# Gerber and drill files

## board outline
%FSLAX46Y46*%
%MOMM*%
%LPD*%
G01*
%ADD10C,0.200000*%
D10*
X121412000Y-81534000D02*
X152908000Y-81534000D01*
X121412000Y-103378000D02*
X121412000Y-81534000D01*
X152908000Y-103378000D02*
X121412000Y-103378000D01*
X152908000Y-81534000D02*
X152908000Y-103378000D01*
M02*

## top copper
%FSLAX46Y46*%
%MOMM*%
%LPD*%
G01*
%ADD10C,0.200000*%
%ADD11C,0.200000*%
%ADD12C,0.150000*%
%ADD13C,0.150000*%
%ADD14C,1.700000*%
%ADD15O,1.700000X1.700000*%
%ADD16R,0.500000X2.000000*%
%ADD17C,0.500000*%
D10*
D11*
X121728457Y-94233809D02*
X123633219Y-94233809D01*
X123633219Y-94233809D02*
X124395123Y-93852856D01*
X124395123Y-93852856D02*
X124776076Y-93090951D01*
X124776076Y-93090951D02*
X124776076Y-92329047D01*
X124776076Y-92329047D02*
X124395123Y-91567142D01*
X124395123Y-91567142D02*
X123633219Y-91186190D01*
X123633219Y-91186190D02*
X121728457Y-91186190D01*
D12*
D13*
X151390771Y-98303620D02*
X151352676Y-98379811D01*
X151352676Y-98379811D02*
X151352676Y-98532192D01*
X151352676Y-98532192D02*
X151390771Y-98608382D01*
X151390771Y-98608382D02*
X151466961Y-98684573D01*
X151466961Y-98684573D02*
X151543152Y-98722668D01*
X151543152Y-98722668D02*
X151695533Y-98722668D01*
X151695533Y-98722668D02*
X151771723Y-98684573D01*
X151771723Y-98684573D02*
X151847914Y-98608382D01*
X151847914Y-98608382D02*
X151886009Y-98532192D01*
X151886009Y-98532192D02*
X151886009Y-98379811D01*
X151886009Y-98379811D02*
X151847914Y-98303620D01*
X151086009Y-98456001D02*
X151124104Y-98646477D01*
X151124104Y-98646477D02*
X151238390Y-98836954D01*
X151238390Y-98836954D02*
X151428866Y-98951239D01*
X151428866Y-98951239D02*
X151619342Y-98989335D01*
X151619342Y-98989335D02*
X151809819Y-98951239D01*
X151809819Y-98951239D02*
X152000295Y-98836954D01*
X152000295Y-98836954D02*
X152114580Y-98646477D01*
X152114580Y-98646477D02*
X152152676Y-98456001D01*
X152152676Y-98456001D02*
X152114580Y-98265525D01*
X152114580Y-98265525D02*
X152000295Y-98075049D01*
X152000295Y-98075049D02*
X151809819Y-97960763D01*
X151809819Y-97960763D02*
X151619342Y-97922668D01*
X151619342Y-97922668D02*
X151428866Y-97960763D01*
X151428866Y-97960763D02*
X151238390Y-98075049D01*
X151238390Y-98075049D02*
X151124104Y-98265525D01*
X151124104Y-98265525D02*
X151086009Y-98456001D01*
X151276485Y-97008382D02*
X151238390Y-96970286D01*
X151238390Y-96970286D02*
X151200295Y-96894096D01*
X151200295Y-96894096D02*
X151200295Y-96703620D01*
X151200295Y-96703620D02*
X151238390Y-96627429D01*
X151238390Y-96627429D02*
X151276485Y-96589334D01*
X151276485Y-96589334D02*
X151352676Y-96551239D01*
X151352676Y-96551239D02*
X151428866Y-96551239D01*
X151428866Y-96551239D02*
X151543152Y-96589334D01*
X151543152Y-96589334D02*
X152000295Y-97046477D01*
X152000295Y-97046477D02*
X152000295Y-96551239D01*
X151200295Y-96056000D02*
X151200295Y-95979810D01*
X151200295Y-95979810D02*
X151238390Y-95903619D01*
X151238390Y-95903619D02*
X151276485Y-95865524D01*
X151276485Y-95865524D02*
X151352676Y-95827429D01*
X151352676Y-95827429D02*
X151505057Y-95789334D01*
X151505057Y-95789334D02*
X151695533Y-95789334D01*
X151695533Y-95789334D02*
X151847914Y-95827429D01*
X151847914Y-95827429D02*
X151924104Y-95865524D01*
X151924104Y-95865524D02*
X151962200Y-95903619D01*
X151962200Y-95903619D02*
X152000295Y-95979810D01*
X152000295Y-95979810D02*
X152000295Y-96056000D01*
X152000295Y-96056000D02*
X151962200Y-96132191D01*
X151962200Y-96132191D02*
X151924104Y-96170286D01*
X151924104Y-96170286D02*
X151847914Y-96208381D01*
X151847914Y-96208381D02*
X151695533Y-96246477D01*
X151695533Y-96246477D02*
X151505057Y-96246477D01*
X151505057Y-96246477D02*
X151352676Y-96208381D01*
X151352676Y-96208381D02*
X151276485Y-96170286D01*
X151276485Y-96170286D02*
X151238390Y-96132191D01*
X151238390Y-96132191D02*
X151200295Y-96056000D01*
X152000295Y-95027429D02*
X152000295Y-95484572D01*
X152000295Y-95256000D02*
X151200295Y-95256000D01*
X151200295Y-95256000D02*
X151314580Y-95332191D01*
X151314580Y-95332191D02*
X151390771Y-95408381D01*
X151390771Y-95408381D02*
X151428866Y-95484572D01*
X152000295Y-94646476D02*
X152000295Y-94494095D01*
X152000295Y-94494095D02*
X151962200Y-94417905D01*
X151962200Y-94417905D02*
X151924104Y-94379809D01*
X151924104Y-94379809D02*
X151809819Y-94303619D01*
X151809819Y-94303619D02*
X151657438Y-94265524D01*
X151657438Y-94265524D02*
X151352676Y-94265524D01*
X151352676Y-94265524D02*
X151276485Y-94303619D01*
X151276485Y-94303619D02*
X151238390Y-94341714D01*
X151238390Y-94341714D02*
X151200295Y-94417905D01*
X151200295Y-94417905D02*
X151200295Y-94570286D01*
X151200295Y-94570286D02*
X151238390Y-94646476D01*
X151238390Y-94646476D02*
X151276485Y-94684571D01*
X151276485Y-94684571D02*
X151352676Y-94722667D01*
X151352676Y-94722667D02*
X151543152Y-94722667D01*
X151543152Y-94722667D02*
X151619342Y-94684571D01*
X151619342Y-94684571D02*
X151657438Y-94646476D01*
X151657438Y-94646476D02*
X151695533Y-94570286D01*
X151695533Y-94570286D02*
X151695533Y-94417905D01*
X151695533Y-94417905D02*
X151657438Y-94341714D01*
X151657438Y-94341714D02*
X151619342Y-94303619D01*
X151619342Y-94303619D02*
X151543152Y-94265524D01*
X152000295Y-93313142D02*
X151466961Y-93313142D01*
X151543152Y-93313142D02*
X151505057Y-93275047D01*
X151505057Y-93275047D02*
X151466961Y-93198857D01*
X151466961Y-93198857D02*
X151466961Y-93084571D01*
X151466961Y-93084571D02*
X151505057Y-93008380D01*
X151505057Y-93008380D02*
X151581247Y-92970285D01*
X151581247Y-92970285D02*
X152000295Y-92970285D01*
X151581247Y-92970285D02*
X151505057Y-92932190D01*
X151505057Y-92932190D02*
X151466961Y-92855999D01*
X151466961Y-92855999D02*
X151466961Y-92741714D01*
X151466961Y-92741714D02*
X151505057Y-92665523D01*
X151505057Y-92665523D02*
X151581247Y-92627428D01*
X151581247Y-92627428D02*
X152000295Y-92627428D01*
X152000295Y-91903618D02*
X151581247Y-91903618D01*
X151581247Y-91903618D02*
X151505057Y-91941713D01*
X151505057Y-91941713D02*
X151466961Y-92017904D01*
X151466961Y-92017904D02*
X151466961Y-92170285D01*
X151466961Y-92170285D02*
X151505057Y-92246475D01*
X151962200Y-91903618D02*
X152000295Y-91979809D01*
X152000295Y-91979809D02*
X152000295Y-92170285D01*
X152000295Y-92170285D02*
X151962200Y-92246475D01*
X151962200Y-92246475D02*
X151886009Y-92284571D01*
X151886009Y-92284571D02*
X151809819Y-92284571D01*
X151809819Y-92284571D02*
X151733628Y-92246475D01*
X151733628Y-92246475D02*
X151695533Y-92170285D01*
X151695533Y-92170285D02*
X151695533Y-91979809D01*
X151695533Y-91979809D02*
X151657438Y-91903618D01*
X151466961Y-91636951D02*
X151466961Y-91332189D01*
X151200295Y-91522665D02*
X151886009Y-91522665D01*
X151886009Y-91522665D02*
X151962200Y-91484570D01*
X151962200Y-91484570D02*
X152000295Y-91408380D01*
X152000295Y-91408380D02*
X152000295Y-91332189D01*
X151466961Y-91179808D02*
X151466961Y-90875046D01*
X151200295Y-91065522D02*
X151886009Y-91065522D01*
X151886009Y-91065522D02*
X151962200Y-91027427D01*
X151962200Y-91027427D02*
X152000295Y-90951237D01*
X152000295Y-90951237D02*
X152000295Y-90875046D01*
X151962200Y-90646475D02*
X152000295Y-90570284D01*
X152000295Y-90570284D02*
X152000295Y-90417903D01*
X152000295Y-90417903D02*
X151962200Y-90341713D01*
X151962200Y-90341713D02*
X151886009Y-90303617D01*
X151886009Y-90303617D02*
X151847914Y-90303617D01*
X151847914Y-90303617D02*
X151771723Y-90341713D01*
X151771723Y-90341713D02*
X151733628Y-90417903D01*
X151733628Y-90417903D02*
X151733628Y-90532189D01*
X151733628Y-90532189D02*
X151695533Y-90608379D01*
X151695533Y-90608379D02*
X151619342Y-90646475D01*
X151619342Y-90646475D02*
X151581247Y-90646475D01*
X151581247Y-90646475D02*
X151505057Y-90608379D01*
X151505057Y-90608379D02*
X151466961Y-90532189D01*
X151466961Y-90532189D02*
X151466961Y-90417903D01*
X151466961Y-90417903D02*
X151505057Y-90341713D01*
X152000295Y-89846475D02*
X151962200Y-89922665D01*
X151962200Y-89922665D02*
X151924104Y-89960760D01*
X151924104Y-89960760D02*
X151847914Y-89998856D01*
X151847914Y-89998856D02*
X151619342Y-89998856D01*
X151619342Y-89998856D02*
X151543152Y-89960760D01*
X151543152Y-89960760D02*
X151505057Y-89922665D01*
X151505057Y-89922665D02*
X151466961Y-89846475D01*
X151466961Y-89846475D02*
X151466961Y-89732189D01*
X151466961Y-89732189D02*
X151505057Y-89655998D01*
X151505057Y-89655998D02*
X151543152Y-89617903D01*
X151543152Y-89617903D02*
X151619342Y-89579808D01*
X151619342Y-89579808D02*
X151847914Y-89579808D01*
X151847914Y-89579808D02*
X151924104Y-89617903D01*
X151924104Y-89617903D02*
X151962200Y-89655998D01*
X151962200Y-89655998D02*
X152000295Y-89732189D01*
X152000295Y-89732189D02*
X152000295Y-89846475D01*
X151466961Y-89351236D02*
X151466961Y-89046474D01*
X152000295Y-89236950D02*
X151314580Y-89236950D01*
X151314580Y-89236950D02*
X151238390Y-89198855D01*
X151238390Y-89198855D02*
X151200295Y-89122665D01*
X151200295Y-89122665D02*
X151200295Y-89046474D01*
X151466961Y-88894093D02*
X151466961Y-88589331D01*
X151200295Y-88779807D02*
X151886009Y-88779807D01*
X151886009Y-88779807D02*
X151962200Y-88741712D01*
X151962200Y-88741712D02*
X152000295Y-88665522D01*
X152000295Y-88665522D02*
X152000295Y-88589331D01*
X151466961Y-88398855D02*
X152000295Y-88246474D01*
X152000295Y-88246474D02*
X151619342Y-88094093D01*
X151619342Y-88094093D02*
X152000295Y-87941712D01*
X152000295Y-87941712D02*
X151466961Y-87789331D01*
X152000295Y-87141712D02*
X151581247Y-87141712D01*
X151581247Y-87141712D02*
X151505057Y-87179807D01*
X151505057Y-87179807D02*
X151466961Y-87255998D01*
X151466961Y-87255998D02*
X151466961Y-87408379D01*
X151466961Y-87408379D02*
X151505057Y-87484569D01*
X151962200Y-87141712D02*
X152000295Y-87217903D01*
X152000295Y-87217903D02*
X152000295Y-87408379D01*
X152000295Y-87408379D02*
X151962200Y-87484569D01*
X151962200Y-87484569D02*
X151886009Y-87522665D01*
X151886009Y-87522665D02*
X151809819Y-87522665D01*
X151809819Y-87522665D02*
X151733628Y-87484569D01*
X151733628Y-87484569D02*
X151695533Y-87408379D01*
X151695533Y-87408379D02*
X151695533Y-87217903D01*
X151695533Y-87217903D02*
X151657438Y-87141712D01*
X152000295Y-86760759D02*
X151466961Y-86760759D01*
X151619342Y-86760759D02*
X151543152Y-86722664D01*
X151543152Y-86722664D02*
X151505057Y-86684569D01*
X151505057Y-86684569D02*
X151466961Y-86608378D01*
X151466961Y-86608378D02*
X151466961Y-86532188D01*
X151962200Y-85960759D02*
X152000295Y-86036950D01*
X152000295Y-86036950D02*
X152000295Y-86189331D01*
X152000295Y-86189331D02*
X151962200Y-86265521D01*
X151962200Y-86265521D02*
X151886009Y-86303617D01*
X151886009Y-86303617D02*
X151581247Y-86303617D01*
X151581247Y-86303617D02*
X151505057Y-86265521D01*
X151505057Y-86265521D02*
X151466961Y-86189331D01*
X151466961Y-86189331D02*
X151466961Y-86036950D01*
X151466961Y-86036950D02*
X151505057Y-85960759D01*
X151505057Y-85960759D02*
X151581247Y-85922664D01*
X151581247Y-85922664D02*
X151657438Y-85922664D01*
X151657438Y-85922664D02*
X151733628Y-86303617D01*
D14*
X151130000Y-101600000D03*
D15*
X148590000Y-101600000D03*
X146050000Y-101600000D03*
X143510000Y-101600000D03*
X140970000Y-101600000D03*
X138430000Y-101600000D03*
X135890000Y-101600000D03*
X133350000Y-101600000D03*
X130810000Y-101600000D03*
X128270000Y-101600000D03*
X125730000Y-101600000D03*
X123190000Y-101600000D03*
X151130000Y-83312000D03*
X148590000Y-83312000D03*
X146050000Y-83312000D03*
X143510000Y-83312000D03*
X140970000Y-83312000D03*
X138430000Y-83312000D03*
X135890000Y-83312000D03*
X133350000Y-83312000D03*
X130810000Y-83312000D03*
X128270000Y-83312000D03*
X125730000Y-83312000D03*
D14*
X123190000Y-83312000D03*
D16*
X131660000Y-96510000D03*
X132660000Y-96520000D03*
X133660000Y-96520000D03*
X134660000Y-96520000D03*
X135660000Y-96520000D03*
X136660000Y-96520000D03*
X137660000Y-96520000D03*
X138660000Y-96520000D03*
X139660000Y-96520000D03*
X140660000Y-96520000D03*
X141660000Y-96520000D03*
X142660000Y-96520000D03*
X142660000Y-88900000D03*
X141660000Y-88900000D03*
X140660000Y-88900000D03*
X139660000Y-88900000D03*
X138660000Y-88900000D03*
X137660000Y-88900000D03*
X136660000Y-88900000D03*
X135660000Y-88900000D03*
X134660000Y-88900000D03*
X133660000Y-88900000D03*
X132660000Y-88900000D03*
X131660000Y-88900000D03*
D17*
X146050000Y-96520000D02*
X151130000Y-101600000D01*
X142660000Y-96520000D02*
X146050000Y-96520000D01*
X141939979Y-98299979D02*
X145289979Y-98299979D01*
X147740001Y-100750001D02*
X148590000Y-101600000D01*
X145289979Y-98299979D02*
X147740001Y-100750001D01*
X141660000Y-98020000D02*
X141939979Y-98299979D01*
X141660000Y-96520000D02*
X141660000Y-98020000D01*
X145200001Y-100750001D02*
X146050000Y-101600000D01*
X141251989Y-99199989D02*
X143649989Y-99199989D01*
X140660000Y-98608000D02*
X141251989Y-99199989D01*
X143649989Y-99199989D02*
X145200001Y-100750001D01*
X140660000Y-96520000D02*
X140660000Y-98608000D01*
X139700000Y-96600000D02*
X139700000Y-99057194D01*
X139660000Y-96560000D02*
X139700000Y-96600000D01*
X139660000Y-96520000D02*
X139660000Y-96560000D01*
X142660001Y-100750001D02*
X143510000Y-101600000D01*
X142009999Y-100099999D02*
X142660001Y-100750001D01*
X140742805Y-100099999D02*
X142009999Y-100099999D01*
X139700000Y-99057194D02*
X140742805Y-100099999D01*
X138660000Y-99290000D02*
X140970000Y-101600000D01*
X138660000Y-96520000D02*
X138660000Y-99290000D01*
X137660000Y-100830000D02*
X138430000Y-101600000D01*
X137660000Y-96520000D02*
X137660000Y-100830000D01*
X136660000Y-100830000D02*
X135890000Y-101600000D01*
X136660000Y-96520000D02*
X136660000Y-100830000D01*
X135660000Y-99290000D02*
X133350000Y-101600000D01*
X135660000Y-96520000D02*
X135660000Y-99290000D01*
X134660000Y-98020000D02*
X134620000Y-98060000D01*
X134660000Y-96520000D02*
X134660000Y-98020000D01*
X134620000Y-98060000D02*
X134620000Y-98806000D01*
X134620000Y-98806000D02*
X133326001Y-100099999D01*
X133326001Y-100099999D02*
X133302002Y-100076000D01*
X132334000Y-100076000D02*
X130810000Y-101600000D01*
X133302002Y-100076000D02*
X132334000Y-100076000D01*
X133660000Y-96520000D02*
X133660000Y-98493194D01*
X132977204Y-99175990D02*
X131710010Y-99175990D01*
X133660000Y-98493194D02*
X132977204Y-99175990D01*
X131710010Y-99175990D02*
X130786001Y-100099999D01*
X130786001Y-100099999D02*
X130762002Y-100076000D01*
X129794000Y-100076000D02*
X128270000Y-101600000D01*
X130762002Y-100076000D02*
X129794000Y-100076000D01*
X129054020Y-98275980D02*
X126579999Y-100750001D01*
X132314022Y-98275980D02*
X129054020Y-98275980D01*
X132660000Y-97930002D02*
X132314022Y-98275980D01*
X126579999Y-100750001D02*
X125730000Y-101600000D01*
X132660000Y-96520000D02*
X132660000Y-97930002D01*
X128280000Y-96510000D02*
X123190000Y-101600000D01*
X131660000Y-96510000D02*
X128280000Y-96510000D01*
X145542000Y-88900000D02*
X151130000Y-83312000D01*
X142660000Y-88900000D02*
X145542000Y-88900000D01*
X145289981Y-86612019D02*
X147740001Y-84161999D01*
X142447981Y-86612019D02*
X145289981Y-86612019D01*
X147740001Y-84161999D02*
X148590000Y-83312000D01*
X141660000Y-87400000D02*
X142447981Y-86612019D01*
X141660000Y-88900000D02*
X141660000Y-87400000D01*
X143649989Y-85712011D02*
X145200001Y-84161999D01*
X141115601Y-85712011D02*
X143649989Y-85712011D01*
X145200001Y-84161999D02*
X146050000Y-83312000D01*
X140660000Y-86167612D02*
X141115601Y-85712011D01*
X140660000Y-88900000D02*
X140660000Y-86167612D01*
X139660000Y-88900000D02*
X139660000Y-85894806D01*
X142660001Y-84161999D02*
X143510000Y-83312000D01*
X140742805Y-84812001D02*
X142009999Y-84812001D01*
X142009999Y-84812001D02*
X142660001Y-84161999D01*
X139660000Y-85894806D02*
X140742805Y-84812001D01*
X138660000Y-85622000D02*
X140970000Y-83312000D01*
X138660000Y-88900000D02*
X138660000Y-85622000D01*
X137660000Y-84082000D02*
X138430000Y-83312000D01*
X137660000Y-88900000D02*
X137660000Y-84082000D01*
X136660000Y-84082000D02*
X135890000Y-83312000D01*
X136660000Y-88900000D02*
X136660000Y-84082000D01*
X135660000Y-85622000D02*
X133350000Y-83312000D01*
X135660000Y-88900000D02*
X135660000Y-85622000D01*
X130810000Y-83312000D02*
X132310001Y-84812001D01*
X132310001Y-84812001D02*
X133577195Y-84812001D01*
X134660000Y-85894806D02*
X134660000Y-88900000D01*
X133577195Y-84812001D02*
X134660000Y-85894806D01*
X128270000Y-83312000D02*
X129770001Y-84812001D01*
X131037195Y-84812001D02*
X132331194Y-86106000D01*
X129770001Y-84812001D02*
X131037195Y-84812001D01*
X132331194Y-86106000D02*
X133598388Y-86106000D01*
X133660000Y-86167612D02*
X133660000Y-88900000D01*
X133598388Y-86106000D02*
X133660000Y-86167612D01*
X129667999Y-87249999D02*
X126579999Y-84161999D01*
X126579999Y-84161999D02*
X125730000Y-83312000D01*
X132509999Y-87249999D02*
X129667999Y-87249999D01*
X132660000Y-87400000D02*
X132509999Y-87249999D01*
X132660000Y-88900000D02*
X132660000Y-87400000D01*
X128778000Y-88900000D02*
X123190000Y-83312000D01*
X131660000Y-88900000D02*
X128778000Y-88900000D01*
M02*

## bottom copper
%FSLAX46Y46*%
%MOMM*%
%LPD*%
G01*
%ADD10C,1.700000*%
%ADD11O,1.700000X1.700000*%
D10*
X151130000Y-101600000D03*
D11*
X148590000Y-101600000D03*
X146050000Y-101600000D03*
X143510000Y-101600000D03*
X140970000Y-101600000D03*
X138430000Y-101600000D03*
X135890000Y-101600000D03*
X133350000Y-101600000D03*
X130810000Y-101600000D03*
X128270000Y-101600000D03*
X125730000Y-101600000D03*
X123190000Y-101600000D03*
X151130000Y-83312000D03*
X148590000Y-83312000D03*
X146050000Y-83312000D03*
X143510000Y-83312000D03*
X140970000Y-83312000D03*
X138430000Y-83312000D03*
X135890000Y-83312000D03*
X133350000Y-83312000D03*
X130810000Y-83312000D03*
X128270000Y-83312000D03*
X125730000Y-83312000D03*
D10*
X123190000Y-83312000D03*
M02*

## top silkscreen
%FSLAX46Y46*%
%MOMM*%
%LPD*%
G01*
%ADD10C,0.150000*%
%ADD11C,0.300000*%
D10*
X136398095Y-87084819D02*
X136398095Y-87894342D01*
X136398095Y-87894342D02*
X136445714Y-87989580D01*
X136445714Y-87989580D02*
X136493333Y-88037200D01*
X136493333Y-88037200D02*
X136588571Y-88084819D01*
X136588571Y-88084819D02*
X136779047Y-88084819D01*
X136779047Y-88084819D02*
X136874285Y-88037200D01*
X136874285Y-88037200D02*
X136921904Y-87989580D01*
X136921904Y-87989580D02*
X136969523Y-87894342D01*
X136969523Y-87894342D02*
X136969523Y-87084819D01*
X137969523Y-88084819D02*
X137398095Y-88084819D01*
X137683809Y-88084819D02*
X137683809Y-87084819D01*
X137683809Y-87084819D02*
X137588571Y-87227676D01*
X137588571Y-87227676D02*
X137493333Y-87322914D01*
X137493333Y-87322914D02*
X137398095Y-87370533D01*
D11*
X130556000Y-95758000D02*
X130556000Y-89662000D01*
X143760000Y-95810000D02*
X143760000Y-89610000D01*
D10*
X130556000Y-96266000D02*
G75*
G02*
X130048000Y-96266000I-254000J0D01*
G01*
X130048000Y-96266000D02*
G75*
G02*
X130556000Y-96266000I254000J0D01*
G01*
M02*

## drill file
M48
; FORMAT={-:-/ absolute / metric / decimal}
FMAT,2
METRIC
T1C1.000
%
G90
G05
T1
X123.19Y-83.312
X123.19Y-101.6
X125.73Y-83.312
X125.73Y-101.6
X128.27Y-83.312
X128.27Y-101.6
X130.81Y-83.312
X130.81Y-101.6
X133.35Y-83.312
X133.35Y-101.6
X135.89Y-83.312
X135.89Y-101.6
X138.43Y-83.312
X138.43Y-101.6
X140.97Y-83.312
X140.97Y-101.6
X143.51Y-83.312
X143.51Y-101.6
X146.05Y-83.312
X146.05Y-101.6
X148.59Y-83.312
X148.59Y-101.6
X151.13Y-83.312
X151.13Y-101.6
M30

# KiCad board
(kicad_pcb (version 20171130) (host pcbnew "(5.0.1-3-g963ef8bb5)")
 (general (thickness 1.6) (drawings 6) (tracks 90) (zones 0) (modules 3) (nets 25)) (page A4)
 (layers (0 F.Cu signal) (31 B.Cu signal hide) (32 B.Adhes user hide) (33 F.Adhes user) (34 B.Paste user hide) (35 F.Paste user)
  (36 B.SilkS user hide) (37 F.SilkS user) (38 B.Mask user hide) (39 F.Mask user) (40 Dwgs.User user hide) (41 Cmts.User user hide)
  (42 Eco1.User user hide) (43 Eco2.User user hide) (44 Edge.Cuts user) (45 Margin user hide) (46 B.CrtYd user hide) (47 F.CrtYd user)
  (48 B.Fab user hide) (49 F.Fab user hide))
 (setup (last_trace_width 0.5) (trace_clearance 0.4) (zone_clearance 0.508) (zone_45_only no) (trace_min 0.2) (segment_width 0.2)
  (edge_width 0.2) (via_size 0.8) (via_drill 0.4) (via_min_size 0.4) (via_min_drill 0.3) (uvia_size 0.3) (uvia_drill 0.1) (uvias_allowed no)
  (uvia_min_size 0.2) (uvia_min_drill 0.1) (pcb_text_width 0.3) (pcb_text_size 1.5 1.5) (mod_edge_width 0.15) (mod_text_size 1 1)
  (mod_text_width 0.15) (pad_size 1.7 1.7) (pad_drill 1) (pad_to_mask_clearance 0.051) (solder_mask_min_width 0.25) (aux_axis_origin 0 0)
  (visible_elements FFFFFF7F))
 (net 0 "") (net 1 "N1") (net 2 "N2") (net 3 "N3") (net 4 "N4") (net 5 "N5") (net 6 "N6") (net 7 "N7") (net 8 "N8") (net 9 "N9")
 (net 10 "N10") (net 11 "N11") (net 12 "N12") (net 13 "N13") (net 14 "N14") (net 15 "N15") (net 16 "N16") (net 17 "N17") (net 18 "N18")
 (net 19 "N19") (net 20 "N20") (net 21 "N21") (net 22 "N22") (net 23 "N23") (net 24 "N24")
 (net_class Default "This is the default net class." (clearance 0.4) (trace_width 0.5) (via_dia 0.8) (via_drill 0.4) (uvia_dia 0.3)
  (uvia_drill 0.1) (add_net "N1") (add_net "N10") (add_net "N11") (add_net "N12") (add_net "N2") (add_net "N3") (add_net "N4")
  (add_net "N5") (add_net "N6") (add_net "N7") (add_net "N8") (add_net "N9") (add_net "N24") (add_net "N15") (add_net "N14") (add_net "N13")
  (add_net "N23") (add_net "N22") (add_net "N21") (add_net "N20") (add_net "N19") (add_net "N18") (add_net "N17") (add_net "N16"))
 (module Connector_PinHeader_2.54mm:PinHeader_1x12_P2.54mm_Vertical (layer B.Cu) (at 151.13 101.6 90)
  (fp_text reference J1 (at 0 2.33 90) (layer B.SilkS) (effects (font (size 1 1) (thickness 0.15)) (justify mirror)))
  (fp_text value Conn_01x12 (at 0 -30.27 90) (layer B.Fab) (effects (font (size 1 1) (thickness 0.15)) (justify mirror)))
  (pad 1 thru_hole circle (at 0 0 90) (size 1.7 1.7) (drill 1) (layers *.Cu *.Mask) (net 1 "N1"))
  (pad 2 thru_hole oval (at 0 -2.54 90) (size 1.7 1.7) (drill 1) (layers *.Cu *.Mask) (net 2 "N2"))
  (pad 3 thru_hole oval (at 0 -5.08 90) (size 1.7 1.7) (drill 1) (layers *.Cu *.Mask) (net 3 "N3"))
  (pad 4 thru_hole oval (at 0 -7.62 90) (size 1.7 1.7) (drill 1) (layers *.Cu *.Mask) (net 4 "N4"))
  (pad 5 thru_hole oval (at 0 -10.16 90) (size 1.7 1.7) (drill 1) (layers *.Cu *.Mask) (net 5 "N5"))
  (pad 6 thru_hole oval (at 0 -12.7 90) (size 1.7 1.7) (drill 1) (layers *.Cu *.Mask) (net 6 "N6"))
  (pad 7 thru_hole oval (at 0 -15.24 90) (size 1.7 1.7) (drill 1) (layers *.Cu *.Mask) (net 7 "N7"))
  (pad 8 thru_hole oval (at 0 -17.78 90) (size 1.7 1.7) (drill 1) (layers *.Cu *.Mask) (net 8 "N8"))
  (pad 9 thru_hole oval (at 0 -20.32 90) (size 1.7 1.7) (drill 1) (layers *.Cu *.Mask) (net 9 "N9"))
  (pad 10 thru_hole oval (at 0 -22.86 90) (size 1.7 1.7) (drill 1) (layers *.Cu *.Mask) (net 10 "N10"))
  (pad 11 thru_hole oval (at 0 -25.4 90) (size 1.7 1.7) (drill 1) (layers *.Cu *.Mask) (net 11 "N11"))
  (pad 12 thru_hole oval (at 0 -27.94 90) (size 1.7 1.7) (drill 1) (layers *.Cu *.Mask) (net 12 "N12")))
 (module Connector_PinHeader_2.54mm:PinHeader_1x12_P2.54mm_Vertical (layer B.Cu) (at 123.19 83.312 270)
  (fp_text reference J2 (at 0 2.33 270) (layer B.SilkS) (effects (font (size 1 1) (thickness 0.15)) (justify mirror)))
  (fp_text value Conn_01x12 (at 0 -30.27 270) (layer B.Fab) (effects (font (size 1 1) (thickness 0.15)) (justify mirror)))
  (pad 12 thru_hole oval (at 0 -27.94 270) (size 1.7 1.7) (drill 1) (layers *.Cu *.Mask) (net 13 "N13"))
  (pad 11 thru_hole oval (at 0 -25.4 270) (size 1.7 1.7) (drill 1) (layers *.Cu *.Mask) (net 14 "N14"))
  (pad 10 thru_hole oval (at 0 -22.86 270) (size 1.7 1.7) (drill 1) (layers *.Cu *.Mask) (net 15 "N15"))
  (pad 9 thru_hole oval (at 0 -20.32 270) (size 1.7 1.7) (drill 1) (layers *.Cu *.Mask) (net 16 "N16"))
  (pad 8 thru_hole oval (at 0 -17.78 270) (size 1.7 1.7) (drill 1) (layers *.Cu *.Mask) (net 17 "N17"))
  (pad 7 thru_hole oval (at 0 -15.24 270) (size 1.7 1.7) (drill 1) (layers *.Cu *.Mask) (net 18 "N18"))
  (pad 6 thru_hole oval (at 0 -12.7 270) (size 1.7 1.7) (drill 1) (layers *.Cu *.Mask) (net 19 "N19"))
  (pad 5 thru_hole oval (at 0 -10.16 270) (size 1.7 1.7) (drill 1) (layers *.Cu *.Mask) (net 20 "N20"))
  (pad 4 thru_hole oval (at 0 -7.62 270) (size 1.7 1.7) (drill 1) (layers *.Cu *.Mask) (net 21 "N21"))
  (pad 3 thru_hole oval (at 0 -5.08 270) (size 1.7 1.7) (drill 1) (layers *.Cu *.Mask) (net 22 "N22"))
  (pad 2 thru_hole oval (at 0 -2.54 270) (size 1.7 1.7) (drill 1) (layers *.Cu *.Mask) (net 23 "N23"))
  (pad 1 thru_hole circle (at 0 0 270) (size 1.7 1.7) (drill 1) (layers *.Cu *.Mask) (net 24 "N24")))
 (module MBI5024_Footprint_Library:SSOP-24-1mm (layer F.Cu) (at 137.16 92.71)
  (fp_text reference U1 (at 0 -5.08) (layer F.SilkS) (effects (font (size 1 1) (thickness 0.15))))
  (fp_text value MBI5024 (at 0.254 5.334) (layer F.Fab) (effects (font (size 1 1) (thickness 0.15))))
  (fp_line (start -6.604 3.048) (end -6.604 -3.048) (layer F.SilkS) (width 0.3))
  (fp_line (start 6.6 3.1) (end 6.6 -3.1) (layer F.SilkS) (width 0.3))
  (fp_circle (center -6.858 3.556) (end -6.858 3.302) (layer F.SilkS) (width 0.15))
  (pad 1 smd rect (at -5.5 3.8) (size 0.5 2) (layers F.Cu F.Paste F.Mask) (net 12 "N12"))
  (pad 2 smd rect (at -4.5 3.81) (size 0.5 2) (layers F.Cu F.Paste F.Mask) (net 11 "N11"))
  (pad 3 smd rect (at -3.5 3.81) (size 0.5 2) (layers F.Cu F.Paste F.Mask) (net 10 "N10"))
  (pad 4 smd rect (at -2.5 3.81) (size 0.5 2) (layers F.Cu F.Paste F.Mask) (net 9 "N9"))
  (pad 5 smd rect (at -1.5 3.81) (size 0.5 2) (layers F.Cu F.Paste F.Mask) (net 8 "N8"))
  (pad 6 smd rect (at -0.5 3.81) (size 0.5 2) (layers F.Cu F.Paste F.Mask) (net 7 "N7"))
  (pad 7 smd rect (at 0.5 3.81) (size 0.5 2) (layers F.Cu F.Paste F.Mask) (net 6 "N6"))
  (pad 8 smd rect (at 1.5 3.81) (size 0.5 2) (layers F.Cu F.Paste F.Mask) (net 5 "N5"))
  (pad 9 smd rect (at 2.5 3.81) (size 0.5 2) (layers F.Cu F.Paste F.Mask) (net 4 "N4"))
  (pad 10 smd rect (at 3.5 3.81) (size 0.5 2) (layers F.Cu F.Paste F.Mask) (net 3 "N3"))
  (pad 11 smd rect (at 4.5 3.81) (size 0.5 2) (layers F.Cu F.Paste F.Mask) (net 2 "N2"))
  (pad 12 smd rect (at 5.5 3.81) (size 0.5 2) (layers F.Cu F.Paste F.Mask) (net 1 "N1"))
  (pad 13 smd rect (at 5.5 -3.81) (size 0.5 2) (layers F.Cu F.Paste F.Mask) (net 13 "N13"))
  (pad 14 smd rect (at 4.5 -3.81) (size 0.5 2) (layers F.Cu F.Paste F.Mask) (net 14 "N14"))
  (pad 15 smd rect (at 3.5 -3.81) (size 0.5 2) (layers F.Cu F.Paste F.Mask) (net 15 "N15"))
  (pad 16 smd rect (at 2.5 -3.81) (size 0.5 2) (layers F.Cu F.Paste F.Mask) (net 16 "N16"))
  (pad 17 smd rect (at 1.5 -3.81) (size 0.5 2) (layers F.Cu F.Paste F.Mask) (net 17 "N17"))
  (pad 18 smd rect (at 0.5 -3.81) (size 0.5 2) (layers F.Cu F.Paste F.Mask) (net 18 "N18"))
  (pad 19 smd rect (at -0.5 -3.81) (size 0.5 2) (layers F.Cu F.Paste F.Mask) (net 19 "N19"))
  (pad 20 smd rect (at -1.5 -3.81) (size 0.5 2) (layers F.Cu F.Paste F.Mask) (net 20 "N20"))
  (pad 21 smd rect (at -2.5 -3.81) (size 0.5 2) (layers F.Cu F.Paste F.Mask) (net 21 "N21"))
  (pad 22 smd rect (at -3.5 -3.81) (size 0.5 2) (layers F.Cu F.Paste F.Mask) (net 22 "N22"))
  (pad 23 smd rect (at -4.5 -3.81) (size 0.5 2) (layers F.Cu F.Paste F.Mask) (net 23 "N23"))
  (pad 24 smd rect (at -5.5 -3.81) (size 0.5 2) (layers F.Cu F.Paste F.Mask) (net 24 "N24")))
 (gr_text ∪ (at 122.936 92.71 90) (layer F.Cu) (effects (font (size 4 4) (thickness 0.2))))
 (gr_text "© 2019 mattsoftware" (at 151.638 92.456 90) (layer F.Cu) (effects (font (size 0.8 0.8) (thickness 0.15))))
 (gr_line (start 121.412 81.534) (end 152.908 81.534) (layer Edge.Cuts) (width 0.2))
 (gr_line (start 121.412 103.378) (end 121.412 81.534) (layer Edge.Cuts) (width 0.2))
 (gr_line (start 152.908 103.378) (end 121.412 103.378) (layer Edge.Cuts) (width 0.2))
 (gr_line (start 152.908 81.534) (end 152.908 103.378) (layer Edge.Cuts) (width 0.2))
 (segment (start 146.05 96.52) (end 151.13 101.6) (width 0.5) (layer F.Cu) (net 1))
 (segment (start 142.66 96.52) (end 146.05 96.52) (width 0.5) (layer F.Cu) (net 1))
 (segment (start 141.939979 98.299979) (end 145.289979 98.299979) (width 0.5) (layer F.Cu) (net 2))
 (segment (start 147.740001 100.750001) (end 148.59 101.6) (width 0.5) (layer F.Cu) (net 2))
 (segment (start 145.289979 98.299979) (end 147.740001 100.750001) (width 0.5) (layer F.Cu) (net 2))
 (segment (start 141.66 98.02) (end 141.939979 98.299979) (width 0.5) (layer F.Cu) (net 2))
 (segment (start 141.66 96.52) (end 141.66 98.02) (width 0.5) (layer F.Cu) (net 2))
 (segment (start 145.200001 100.750001) (end 146.05 101.6) (width 0.5) (layer F.Cu) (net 3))
 (segment (start 141.251989 99.199989) (end 143.649989 99.199989) (width 0.5) (layer F.Cu) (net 3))
 (segment (start 140.66 98.608) (end 141.251989 99.199989) (width 0.5) (layer F.Cu) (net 3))
 (segment (start 143.649989 99.199989) (end 145.200001 100.750001) (width 0.5) (layer F.Cu) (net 3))
 (segment (start 140.66 96.52) (end 140.66 98.608) (width 0.5) (layer F.Cu) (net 3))
 (segment (start 139.7 96.6) (end 139.7 99.057194) (width 0.5) (layer F.Cu) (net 4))
 (segment (start 139.66 96.56) (end 139.7 96.6) (width 0.5) (layer F.Cu) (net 4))
 (segment (start 139.66 96.52) (end 139.66 96.56) (width 0.5) (layer F.Cu) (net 4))
 (segment (start 142.660001 100.750001) (end 143.51 101.6) (width 0.5) (layer F.Cu) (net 4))
 (segment (start 142.009999 100.099999) (end 142.660001 100.750001) (width 0.5) (layer F.Cu) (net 4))
 (segment (start 140.742805 100.099999) (end 142.009999 100.099999) (width 0.5) (layer F.Cu) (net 4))
 (segment (start 139.7 99.057194) (end 140.742805 100.099999) (width 0.5) (layer F.Cu) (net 4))
 (segment (start 138.66 99.29) (end 140.97 101.6) (width 0.5) (layer F.Cu) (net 5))
 (segment (start 138.66 96.52) (end 138.66 99.29) (width 0.5) (layer F.Cu) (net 5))
 (segment (start 137.66 100.83) (end 138.43 101.6) (width 0.5) (layer F.Cu) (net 6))
 (segment (start 137.66 96.52) (end 137.66 100.83) (width 0.5) (layer F.Cu) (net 6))
 (segment (start 136.66 100.83) (end 135.89 101.6) (width 0.5) (layer F.Cu) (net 7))
 (segment (start 136.66 96.52) (end 136.66 100.83) (width 0.5) (layer F.Cu) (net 7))
 (segment (start 135.66 99.29) (end 133.35 101.6) (width 0.5) (layer F.Cu) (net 8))
 (segment (start 135.66 96.52) (end 135.66 99.29) (width 0.5) (layer F.Cu) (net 8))
 (segment (start 134.66 98.02) (end 134.62 98.06) (width 0.5) (layer F.Cu) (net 9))
 (segment (start 134.66 96.52) (end 134.66 98.02) (width 0.5) (layer F.Cu) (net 9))
 (segment (start 134.62 98.06) (end 134.62 98.806) (width 0.5) (layer F.Cu) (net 9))
 (segment (start 134.62 98.806) (end 133.326001 100.099999) (width 0.5) (layer F.Cu) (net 9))
 (segment (start 133.326001 100.099999) (end 133.302002 100.076) (width 0.5) (layer F.Cu) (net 9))
 (segment (start 132.334 100.076) (end 130.81 101.6) (width 0.5) (layer F.Cu) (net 9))
 (segment (start 133.302002 100.076) (end 132.334 100.076) (width 0.5) (layer F.Cu) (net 9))
 (segment (start 133.66 96.52) (end 133.66 98.493194) (width 0.5) (layer F.Cu) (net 10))
 (segment (start 132.977204 99.17599) (end 131.71001 99.17599) (width 0.5) (layer F.Cu) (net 10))
 (segment (start 133.66 98.493194) (end 132.977204 99.17599) (width 0.5) (layer F.Cu) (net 10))
 (segment (start 131.71001 99.17599) (end 130.786001 100.099999) (width 0.5) (layer F.Cu) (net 10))
 (segment (start 130.786001 100.099999) (end 130.762002 100.076) (width 0.5) (layer F.Cu) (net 10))
 (segment (start 129.794 100.076) (end 128.27 101.6) (width 0.5) (layer F.Cu) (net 10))
 (segment (start 130.762002 100.076) (end 129.794 100.076) (width 0.5) (layer F.Cu) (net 10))
 (segment (start 129.05402 98.27598) (end 126.579999 100.750001) (width 0.5) (layer F.Cu) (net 11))
 (segment (start 132.314022 98.27598) (end 129.05402 98.27598) (width 0.5) (layer F.Cu) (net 11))
 (segment (start 132.66 97.930002) (end 132.314022 98.27598) (width 0.5) (layer F.Cu) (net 11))
 (segment (start 126.579999 100.750001) (end 125.73 101.6) (width 0.5) (layer F.Cu) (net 11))
 (segment (start 132.66 96.52) (end 132.66 97.930002) (width 0.5) (layer F.Cu) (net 11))
 (segment (start 128.28 96.51) (end 123.19 101.6) (width 0.5) (layer F.Cu) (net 12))
 (segment (start 131.66 96.51) (end 128.28 96.51) (width 0.5) (layer F.Cu) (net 12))
 (segment (start 145.542 88.9) (end 151.13 83.312) (width 0.5) (layer F.Cu) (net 13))
 (segment (start 142.66 88.9) (end 145.542 88.9) (width 0.5) (layer F.Cu) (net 13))
 (segment (start 145.289981 86.612019) (end 147.740001 84.161999) (width 0.5) (layer F.Cu) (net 14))
 (segment (start 142.447981 86.612019) (end 145.289981 86.612019) (width 0.5) (layer F.Cu) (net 14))
 (segment (start 147.740001 84.161999) (end 148.59 83.312) (width 0.5) (layer F.Cu) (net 14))
 (segment (start 141.66 87.4) (end 142.447981 86.612019) (width 0.5) (layer F.Cu) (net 14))
 (segment (start 141.66 88.9) (end 141.66 87.4) (width 0.5) (layer F.Cu) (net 14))
 (segment (start 143.649989 85.712011) (end 145.200001 84.161999) (width 0.5) (layer F.Cu) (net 15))
 (segment (start 141.115601 85.712011) (end 143.649989 85.712011) (width 0.5) (layer F.Cu) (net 15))
 (segment (start 145.200001 84.161999) (end 146.05 83.312) (width 0.5) (layer F.Cu) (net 15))
 (segment (start 140.66 86.167612) (end 141.115601 85.712011) (width 0.5) (layer F.Cu) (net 15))
 (segment (start 140.66 88.9) (end 140.66 86.167612) (width 0.5) (layer F.Cu) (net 15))
 (segment (start 139.66 88.9) (end 139.66 85.894806) (width 0.5) (layer F.Cu) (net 16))
 (segment (start 142.660001 84.161999) (end 143.51 83.312) (width 0.5) (layer F.Cu) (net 16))
 (segment (start 140.742805 84.812001) (end 142.009999 84.812001) (width 0.5) (layer F.Cu) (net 16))
 (segment (start 142.009999 84.812001) (end 142.660001 84.161999) (width 0.5) (layer F.Cu) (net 16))
 (segment (start 139.66 85.894806) (end 140.742805 84.812001) (width 0.5) (layer F.Cu) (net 16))
 (segment (start 138.66 85.622) (end 140.97 83.312) (width 0.5) (layer F.Cu) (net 17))
 (segment (start 138.66 88.9) (end 138.66 85.622) (width 0.5) (layer F.Cu) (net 17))
 (segment (start 137.66 84.082) (end 138.43 83.312) (width 0.5) (layer F.Cu) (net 18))
 (segment (start 137.66 88.9) (end 137.66 84.082) (width 0.5) (layer F.Cu) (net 18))
 (segment (start 136.66 84.082) (end 135.89 83.312) (width 0.5) (layer F.Cu) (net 19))
 (segment (start 136.66 88.9) (end 136.66 84.082) (width 0.5) (layer F.Cu) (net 19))
 (segment (start 135.66 85.622) (end 133.35 83.312) (width 0.5) (layer F.Cu) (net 20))
 (segment (start 135.66 88.9) (end 135.66 85.622) (width 0.5) (layer F.Cu) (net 20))
 (segment (start 130.81 83.312) (end 132.310001 84.812001) (width 0.5) (layer F.Cu) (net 21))
 (segment (start 132.310001 84.812001) (end 133.577195 84.812001) (width 0.5) (layer F.Cu) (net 21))
 (segment (start 134.66 85.894806) (end 134.66 88.9) (width 0.5) (layer F.Cu) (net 21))
 (segment (start 133.577195 84.812001) (end 134.66 85.894806) (width 0.5) (layer F.Cu) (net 21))
 (segment (start 128.27 83.312) (end 129.770001 84.812001) (width 0.5) (layer F.Cu) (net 22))
 (segment (start 131.037195 84.812001) (end 132.331194 86.106) (width 0.5) (layer F.Cu) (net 22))
 (segment (start 129.770001 84.812001) (end 131.037195 84.812001) (width 0.5) (layer F.Cu) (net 22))
 (segment (start 132.331194 86.106) (end 133.598388 86.106) (width 0.5) (layer F.Cu) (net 22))
 (segment (start 133.66 86.167612) (end 133.66 88.9) (width 0.5) (layer F.Cu) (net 22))
 (segment (start 133.598388 86.106) (end 133.66 86.167612) (width 0.5) (layer F.Cu) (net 22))
 (segment (start 129.667999 87.249999) (end 126.579999 84.161999) (width 0.5) (layer F.Cu) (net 23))
 (segment (start 126.579999 84.161999) (end 125.73 83.312) (width 0.5) (layer F.Cu) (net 23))
 (segment (start 132.509999 87.249999) (end 129.667999 87.249999) (width 0.5) (layer F.Cu) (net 23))
 (segment (start 132.66 87.4) (end 132.509999 87.249999) (width 0.5) (layer F.Cu) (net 23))
 (segment (start 132.66 88.9) (end 132.66 87.4) (width 0.5) (layer F.Cu) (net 23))
 (segment (start 128.778 88.9) (end 123.19 83.312) (width 0.5) (layer F.Cu) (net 24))
 (segment (start 131.66 88.9) (end 128.778 88.9) (width 0.5) (layer F.Cu) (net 24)))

